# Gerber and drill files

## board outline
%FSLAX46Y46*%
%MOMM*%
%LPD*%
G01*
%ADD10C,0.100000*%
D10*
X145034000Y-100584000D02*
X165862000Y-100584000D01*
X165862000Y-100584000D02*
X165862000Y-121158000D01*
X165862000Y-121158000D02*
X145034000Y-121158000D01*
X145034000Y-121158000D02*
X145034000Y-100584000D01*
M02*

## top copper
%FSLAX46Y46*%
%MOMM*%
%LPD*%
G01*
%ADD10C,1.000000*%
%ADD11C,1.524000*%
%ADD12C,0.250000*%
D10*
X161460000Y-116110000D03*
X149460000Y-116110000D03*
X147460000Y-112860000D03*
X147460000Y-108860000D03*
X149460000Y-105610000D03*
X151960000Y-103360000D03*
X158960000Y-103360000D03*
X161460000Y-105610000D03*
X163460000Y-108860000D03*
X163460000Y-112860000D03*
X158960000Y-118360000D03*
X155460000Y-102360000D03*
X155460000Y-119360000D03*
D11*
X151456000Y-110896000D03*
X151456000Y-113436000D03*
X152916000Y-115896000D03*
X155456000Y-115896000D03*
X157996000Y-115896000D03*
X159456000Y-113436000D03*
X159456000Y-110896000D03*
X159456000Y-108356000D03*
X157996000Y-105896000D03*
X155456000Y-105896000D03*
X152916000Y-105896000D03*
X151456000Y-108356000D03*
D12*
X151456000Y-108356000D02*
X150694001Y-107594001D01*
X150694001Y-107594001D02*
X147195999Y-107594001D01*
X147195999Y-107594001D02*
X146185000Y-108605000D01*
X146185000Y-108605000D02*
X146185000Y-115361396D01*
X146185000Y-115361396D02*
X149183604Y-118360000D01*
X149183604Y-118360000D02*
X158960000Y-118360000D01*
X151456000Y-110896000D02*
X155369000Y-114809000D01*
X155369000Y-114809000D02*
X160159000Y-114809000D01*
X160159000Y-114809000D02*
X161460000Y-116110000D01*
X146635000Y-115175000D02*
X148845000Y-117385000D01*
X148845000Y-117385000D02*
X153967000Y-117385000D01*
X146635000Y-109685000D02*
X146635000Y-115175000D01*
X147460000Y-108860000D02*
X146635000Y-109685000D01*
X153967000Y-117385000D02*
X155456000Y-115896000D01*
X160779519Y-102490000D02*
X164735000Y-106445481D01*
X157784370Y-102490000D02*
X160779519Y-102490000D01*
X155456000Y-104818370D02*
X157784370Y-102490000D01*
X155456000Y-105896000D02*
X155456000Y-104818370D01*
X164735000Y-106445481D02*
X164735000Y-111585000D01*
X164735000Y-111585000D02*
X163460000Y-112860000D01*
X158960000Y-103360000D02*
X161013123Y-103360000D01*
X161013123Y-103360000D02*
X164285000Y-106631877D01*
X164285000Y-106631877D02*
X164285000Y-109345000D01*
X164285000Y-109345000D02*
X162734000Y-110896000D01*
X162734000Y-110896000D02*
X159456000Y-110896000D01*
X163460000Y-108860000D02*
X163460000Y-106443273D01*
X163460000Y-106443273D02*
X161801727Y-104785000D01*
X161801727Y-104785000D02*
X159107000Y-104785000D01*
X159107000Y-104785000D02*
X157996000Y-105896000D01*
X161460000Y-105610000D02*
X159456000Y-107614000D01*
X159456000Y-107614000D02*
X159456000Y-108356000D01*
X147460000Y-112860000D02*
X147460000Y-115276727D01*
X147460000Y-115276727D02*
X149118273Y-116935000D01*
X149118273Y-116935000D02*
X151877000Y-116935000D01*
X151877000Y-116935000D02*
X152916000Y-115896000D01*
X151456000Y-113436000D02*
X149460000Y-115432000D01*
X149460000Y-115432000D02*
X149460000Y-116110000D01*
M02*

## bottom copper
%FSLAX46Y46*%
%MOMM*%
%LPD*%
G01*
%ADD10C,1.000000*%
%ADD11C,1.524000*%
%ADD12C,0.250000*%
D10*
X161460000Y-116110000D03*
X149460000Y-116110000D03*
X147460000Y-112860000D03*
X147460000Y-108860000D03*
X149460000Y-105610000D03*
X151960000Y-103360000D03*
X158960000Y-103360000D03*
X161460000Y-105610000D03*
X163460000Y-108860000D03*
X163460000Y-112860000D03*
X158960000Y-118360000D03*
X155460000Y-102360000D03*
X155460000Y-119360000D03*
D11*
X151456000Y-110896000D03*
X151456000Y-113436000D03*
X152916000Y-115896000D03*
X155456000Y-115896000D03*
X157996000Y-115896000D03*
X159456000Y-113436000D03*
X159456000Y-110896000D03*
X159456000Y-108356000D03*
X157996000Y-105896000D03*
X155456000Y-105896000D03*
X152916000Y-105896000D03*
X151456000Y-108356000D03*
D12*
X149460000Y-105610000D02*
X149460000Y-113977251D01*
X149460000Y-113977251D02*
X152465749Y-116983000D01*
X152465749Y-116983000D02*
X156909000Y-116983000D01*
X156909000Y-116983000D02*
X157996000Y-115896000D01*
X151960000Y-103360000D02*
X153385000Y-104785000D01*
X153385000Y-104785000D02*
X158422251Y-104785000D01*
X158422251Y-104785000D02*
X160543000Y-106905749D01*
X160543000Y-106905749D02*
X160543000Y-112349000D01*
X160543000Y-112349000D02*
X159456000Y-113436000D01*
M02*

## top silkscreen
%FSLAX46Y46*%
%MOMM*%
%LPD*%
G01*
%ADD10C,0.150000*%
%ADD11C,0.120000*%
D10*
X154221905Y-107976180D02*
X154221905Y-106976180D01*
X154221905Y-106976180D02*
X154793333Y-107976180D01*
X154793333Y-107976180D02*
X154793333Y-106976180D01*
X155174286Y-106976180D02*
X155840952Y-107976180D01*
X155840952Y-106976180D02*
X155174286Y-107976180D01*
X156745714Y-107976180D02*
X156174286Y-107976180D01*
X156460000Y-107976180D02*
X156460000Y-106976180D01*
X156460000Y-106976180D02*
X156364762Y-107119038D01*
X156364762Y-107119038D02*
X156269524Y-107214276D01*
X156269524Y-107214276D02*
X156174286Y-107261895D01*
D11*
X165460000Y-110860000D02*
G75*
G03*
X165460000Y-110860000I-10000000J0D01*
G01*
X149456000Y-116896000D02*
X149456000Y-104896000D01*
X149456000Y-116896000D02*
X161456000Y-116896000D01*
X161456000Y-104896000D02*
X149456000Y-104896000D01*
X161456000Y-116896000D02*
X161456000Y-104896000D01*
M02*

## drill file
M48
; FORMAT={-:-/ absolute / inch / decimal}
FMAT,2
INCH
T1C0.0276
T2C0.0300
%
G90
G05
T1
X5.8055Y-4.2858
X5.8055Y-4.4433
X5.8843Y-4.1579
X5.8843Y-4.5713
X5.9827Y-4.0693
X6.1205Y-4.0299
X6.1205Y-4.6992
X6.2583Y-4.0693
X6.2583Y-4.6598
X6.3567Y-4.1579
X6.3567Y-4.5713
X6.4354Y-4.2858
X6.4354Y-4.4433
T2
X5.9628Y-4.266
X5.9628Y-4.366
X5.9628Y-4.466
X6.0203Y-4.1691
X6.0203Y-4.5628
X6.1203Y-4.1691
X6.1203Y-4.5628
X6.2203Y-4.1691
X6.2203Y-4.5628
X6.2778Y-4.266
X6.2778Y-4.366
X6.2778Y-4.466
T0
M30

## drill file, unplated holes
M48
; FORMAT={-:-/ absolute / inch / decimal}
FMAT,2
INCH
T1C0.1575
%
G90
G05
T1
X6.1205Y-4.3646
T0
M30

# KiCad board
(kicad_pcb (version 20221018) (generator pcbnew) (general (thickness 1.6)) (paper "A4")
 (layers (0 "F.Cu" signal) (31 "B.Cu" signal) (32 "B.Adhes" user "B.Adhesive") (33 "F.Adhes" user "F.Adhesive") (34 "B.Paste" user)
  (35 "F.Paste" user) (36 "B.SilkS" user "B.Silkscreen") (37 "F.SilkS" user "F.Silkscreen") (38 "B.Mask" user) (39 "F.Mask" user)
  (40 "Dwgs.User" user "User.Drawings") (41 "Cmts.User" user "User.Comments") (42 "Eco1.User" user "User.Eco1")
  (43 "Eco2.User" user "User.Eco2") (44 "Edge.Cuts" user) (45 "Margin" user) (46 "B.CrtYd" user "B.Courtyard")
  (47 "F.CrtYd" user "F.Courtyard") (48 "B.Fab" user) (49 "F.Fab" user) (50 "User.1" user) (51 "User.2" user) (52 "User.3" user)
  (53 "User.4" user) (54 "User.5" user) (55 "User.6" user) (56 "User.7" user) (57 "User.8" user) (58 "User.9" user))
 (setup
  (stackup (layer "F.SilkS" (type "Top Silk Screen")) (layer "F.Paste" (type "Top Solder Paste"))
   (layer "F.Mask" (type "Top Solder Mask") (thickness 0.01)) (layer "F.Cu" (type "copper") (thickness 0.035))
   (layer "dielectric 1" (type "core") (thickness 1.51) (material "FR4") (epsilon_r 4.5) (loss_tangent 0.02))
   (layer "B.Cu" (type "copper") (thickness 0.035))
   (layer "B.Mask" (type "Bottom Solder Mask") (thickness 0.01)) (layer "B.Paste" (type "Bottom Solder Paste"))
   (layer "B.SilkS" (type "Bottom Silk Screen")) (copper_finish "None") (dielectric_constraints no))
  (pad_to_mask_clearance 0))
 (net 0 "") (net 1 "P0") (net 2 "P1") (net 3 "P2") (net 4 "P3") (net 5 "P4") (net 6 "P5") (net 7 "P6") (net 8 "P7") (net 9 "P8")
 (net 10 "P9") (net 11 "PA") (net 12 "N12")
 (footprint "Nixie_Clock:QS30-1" (layer "F.Cu") (at 155.46 110.86)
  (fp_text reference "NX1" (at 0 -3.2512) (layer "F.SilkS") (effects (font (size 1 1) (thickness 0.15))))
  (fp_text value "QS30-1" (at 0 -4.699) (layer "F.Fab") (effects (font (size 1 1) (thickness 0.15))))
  (fp_circle (center 0 0) (end 10 0) (stroke (width 0.12) (type solid)) (fill none) (layer "F.SilkS"))
  (pad "" np_thru_hole circle (at 0 0) (size 4 4) (drill 4) (layers "*.Cu" "*.Mask"))
  (pad "0" thru_hole circle (at 6 5.25) (size 1 1) (drill 0.7) (layers "*.Cu" "*.Mask") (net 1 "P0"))
  (pad "1" thru_hole circle (at -6 5.25) (size 1 1) (drill 0.7) (layers "*.Cu" "*.Mask") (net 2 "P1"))
  (pad "2" thru_hole circle (at -8 2) (size 1 1) (drill 0.7) (layers "*.Cu" "*.Mask") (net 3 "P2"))
  (pad "3" thru_hole circle (at -8 -2) (size 1 1) (drill 0.7) (layers "*.Cu" "*.Mask") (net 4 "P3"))
  (pad "4" thru_hole circle (at -6 -5.25) (size 1 1) (drill 0.7) (layers "*.Cu" "*.Mask") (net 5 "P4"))
  (pad "5" thru_hole circle (at -3.5 -7.5) (size 1 1) (drill 0.7) (layers "*.Cu" "*.Mask") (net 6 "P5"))
  (pad "6" thru_hole circle (at 3.5 -7.5) (size 1 1) (drill 0.7) (layers "*.Cu" "*.Mask") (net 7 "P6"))
  (pad "7" thru_hole circle (at 6 -5.25) (size 1 1) (drill 0.7) (layers "*.Cu" "*.Mask") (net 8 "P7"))
  (pad "8" thru_hole circle (at 8 -2) (size 1 1) (drill 0.7) (layers "*.Cu" "*.Mask") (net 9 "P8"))
  (pad "9" thru_hole circle (at 8 2) (size 1 1) (drill 0.7) (layers "*.Cu" "*.Mask") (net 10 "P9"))
  (pad "A" thru_hole circle (at 3.5 7.5) (size 1 1) (drill 0.7) (layers "*.Cu" "*.Mask") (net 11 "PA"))
  (pad "NC" thru_hole circle (at 0 -8.5) (size 1 1) (drill 0.7) (layers "*.Cu" "*.Mask"))
  (pad "NC" thru_hole circle (at 0 8.5) (size 1 1) (drill 0.7) (layers "*.Cu" "*.Mask")))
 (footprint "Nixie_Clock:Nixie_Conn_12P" (layer "F.Cu") (at 155.456 110.896)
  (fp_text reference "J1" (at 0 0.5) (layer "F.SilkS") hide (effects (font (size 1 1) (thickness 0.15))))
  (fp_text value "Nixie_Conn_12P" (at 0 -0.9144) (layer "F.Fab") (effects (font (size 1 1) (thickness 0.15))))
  (fp_line (start -6 6) (end -6 -6) (stroke (width 0.12) (type solid)) (layer "F.SilkS"))
  (fp_line (start -6 6) (end 6 6) (stroke (width 0.12) (type solid)) (layer "F.SilkS"))
  (fp_line (start 6 -6) (end -6 -6) (stroke (width 0.12) (type solid)) (layer "F.SilkS"))
  (fp_line (start 6 6) (end 6 -6) (stroke (width 0.12) (type solid)) (layer "F.SilkS"))
  (pad "0" thru_hole circle (at -4 0) (size 1.524 1.524) (drill 0.762) (layers "*.Cu" "*.Mask") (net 1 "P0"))
  (pad "1" thru_hole circle (at -4 2.54) (size 1.524 1.524) (drill 0.762) (layers "*.Cu" "*.Mask") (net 2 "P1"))
  (pad "2" thru_hole circle (at -2.54 5) (size 1.524 1.524) (drill 0.762) (layers "*.Cu" "*.Mask") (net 3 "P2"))
  (pad "3" thru_hole circle (at 0 5) (size 1.524 1.524) (drill 0.762) (layers "*.Cu" "*.Mask") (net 4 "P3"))
  (pad "4" thru_hole circle (at 2.54 5) (size 1.524 1.524) (drill 0.762) (layers "*.Cu" "*.Mask") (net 5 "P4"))
  (pad "5" thru_hole circle (at 4 2.54) (size 1.524 1.524) (drill 0.762) (layers "*.Cu" "*.Mask") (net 6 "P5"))
  (pad "6" thru_hole circle (at 4 0) (size 1.524 1.524) (drill 0.762) (layers "*.Cu" "*.Mask") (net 7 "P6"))
  (pad "7" thru_hole circle (at 4 -2.54) (size 1.524 1.524) (drill 0.762) (layers "*.Cu" "*.Mask") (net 8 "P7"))
  (pad "8" thru_hole circle (at 2.54 -5) (size 1.524 1.524) (drill 0.762) (layers "*.Cu" "*.Mask") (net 9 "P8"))
  (pad "9" thru_hole circle (at 0 -5) (size 1.524 1.524) (drill 0.762) (layers "*.Cu" "*.Mask") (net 10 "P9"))
  (pad "10" thru_hole circle (at -2.54 -5) (size 1.524 1.524) (drill 0.762) (layers "*.Cu" "*.Mask") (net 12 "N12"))
  (pad "A" thru_hole circle (at -4 -2.54) (size 1.524 1.524) (drill 0.762) (layers "*.Cu" "*.Mask") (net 11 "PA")))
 (gr_rect (start 145.034 100.584) (end 165.862 121.158) (stroke (width 0.1) (type default)) (fill none) (layer "Edge.Cuts"))
 (segment (start 146.185 108.605) (end 146.185 115.361396) (width 0.25) (layer "F.Cu") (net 11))
 (segment (start 149.183604 118.36) (end 158.96 118.36) (width 0.25) (layer "F.Cu") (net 11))
 (segment (start 150.694001 107.594001) (end 147.195999 107.594001) (width 0.25) (layer "F.Cu") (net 11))
 (segment (start 147.195999 107.594001) (end 146.185 108.605) (width 0.25) (layer "F.Cu") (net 11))
 (segment (start 146.185 115.361396) (end 149.183604 118.36) (width 0.25) (layer "F.Cu") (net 11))
 (segment (start 151.456 108.356) (end 150.694001 107.594001) (width 0.25) (layer "F.Cu") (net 11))
 (segment (start 151.456 110.896) (end 155.369 114.809) (width 0.25) (layer "F.Cu") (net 1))
 (segment (start 160.159 114.809) (end 161.46 116.11) (width 0.25) (layer "F.Cu") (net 1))
 (segment (start 155.369 114.809) (end 160.159 114.809) (width 0.25) (layer "F.Cu") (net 1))
 (segment (start 151.456 113.436) (end 149.46 115.432) (width 0.25) (layer "F.Cu") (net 2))
 (segment (start 149.46 115.432) (end 149.46 116.11) (width 0.25) (layer "F.Cu") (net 2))
 (segment (start 147.46 115.276727) (end 149.118273 116.935) (width 0.25) (layer "F.Cu") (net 3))
 (segment (start 147.46 112.86) (end 147.46 115.276727) (width 0.25) (layer "F.Cu") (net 3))
 (segment (start 151.877 116.935) (end 152.916 115.896) (width 0.25) (layer "F.Cu") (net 3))
 (segment (start 149.118273 116.935) (end 151.877 116.935) (width 0.25) (layer "F.Cu") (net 3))
 (segment (start 146.635 109.685) (end 146.635 115.175) (width 0.25) (layer "F.Cu") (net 4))
 (segment (start 147.46 108.86) (end 146.635 109.685) (width 0.25) (layer "F.Cu") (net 4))
 (segment (start 153.967 117.385) (end 155.456 115.896) (width 0.25) (layer "F.Cu") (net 4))
 (segment (start 146.635 115.175) (end 148.845 117.385) (width 0.25) (layer "F.Cu") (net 4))
 (segment (start 148.845 117.385) (end 153.967 117.385) (width 0.25) (layer "F.Cu") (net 4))
 (segment (start 152.465749 116.983) (end 156.909 116.983) (width 0.25) (layer "B.Cu") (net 5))
 (segment (start 156.909 116.983) (end 157.996 115.896) (width 0.25) (layer "B.Cu") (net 5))
 (segment (start 149.46 105.61) (end 149.46 113.977251) (width 0.25) (layer "B.Cu") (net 5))
 (segment (start 149.46 113.977251) (end 152.465749 116.983) (width 0.25) (layer "B.Cu") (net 5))
 (segment (start 151.96 103.36) (end 153.385 104.785) (width 0.25) (layer "B.Cu") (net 6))
 (segment (start 158.422251 104.785) (end 160.543 106.905749) (width 0.25) (layer "B.Cu") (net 6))
 (segment (start 153.385 104.785) (end 158.422251 104.785) (width 0.25) (layer "B.Cu") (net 6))
 (segment (start 160.543 112.349) (end 159.456 113.436) (width 0.25) (layer "B.Cu") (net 6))
 (segment (start 160.543 106.905749) (end 160.543 112.349) (width 0.25) (layer "B.Cu") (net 6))
 (segment (start 164.285 109.345) (end 162.734 110.896) (width 0.25) (layer "F.Cu") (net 7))
 (segment (start 162.734 110.896) (end 159.456 110.896) (width 0.25) (layer "F.Cu") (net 7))
 (segment (start 158.96 103.36) (end 161.013123 103.36) (width 0.25) (layer "F.Cu") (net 7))
 (segment (start 161.013123 103.36) (end 164.285 106.631877) (width 0.25) (layer "F.Cu") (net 7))
 (segment (start 164.285 106.631877) (end 164.285 109.345) (width 0.25) (layer "F.Cu") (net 7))
 (segment (start 159.456 107.614) (end 159.456 108.356) (width 0.25) (layer "F.Cu") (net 8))
 (segment (start 161.46 105.61) (end 159.456 107.614) (width 0.25) (layer "F.Cu") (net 8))
 (segment (start 163.46 108.86) (end 163.46 106.443273) (width 0.25) (layer "F.Cu") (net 9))
 (segment (start 159.107 104.785) (end 157.996 105.896) (width 0.25) (layer "F.Cu") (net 9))
 (segment (start 163.46 106.443273) (end 161.801727 104.785) (width 0.25) (layer "F.Cu") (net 9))
 (segment (start 161.801727 104.785) (end 159.107 104.785) (width 0.25) (layer "F.Cu") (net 9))
 (segment (start 164.735 111.585) (end 163.46 112.86) (width 0.25) (layer "F.Cu") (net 10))
 (segment (start 157.78437 102.49) (end 160.779519 102.49) (width 0.25) (layer "F.Cu") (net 10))
 (segment (start 164.735 106.445481) (end 164.735 111.585) (width 0.25) (layer "F.Cu") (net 10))
 (segment (start 155.456 104.81837) (end 157.78437 102.49) (width 0.25) (layer "F.Cu") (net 10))
 (segment (start 155.456 105.896) (end 155.456 104.81837) (width 0.25) (layer "F.Cu") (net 10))
 (segment (start 160.779519 102.49) (end 164.735 106.445481) (width 0.25) (layer "F.Cu") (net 10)))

